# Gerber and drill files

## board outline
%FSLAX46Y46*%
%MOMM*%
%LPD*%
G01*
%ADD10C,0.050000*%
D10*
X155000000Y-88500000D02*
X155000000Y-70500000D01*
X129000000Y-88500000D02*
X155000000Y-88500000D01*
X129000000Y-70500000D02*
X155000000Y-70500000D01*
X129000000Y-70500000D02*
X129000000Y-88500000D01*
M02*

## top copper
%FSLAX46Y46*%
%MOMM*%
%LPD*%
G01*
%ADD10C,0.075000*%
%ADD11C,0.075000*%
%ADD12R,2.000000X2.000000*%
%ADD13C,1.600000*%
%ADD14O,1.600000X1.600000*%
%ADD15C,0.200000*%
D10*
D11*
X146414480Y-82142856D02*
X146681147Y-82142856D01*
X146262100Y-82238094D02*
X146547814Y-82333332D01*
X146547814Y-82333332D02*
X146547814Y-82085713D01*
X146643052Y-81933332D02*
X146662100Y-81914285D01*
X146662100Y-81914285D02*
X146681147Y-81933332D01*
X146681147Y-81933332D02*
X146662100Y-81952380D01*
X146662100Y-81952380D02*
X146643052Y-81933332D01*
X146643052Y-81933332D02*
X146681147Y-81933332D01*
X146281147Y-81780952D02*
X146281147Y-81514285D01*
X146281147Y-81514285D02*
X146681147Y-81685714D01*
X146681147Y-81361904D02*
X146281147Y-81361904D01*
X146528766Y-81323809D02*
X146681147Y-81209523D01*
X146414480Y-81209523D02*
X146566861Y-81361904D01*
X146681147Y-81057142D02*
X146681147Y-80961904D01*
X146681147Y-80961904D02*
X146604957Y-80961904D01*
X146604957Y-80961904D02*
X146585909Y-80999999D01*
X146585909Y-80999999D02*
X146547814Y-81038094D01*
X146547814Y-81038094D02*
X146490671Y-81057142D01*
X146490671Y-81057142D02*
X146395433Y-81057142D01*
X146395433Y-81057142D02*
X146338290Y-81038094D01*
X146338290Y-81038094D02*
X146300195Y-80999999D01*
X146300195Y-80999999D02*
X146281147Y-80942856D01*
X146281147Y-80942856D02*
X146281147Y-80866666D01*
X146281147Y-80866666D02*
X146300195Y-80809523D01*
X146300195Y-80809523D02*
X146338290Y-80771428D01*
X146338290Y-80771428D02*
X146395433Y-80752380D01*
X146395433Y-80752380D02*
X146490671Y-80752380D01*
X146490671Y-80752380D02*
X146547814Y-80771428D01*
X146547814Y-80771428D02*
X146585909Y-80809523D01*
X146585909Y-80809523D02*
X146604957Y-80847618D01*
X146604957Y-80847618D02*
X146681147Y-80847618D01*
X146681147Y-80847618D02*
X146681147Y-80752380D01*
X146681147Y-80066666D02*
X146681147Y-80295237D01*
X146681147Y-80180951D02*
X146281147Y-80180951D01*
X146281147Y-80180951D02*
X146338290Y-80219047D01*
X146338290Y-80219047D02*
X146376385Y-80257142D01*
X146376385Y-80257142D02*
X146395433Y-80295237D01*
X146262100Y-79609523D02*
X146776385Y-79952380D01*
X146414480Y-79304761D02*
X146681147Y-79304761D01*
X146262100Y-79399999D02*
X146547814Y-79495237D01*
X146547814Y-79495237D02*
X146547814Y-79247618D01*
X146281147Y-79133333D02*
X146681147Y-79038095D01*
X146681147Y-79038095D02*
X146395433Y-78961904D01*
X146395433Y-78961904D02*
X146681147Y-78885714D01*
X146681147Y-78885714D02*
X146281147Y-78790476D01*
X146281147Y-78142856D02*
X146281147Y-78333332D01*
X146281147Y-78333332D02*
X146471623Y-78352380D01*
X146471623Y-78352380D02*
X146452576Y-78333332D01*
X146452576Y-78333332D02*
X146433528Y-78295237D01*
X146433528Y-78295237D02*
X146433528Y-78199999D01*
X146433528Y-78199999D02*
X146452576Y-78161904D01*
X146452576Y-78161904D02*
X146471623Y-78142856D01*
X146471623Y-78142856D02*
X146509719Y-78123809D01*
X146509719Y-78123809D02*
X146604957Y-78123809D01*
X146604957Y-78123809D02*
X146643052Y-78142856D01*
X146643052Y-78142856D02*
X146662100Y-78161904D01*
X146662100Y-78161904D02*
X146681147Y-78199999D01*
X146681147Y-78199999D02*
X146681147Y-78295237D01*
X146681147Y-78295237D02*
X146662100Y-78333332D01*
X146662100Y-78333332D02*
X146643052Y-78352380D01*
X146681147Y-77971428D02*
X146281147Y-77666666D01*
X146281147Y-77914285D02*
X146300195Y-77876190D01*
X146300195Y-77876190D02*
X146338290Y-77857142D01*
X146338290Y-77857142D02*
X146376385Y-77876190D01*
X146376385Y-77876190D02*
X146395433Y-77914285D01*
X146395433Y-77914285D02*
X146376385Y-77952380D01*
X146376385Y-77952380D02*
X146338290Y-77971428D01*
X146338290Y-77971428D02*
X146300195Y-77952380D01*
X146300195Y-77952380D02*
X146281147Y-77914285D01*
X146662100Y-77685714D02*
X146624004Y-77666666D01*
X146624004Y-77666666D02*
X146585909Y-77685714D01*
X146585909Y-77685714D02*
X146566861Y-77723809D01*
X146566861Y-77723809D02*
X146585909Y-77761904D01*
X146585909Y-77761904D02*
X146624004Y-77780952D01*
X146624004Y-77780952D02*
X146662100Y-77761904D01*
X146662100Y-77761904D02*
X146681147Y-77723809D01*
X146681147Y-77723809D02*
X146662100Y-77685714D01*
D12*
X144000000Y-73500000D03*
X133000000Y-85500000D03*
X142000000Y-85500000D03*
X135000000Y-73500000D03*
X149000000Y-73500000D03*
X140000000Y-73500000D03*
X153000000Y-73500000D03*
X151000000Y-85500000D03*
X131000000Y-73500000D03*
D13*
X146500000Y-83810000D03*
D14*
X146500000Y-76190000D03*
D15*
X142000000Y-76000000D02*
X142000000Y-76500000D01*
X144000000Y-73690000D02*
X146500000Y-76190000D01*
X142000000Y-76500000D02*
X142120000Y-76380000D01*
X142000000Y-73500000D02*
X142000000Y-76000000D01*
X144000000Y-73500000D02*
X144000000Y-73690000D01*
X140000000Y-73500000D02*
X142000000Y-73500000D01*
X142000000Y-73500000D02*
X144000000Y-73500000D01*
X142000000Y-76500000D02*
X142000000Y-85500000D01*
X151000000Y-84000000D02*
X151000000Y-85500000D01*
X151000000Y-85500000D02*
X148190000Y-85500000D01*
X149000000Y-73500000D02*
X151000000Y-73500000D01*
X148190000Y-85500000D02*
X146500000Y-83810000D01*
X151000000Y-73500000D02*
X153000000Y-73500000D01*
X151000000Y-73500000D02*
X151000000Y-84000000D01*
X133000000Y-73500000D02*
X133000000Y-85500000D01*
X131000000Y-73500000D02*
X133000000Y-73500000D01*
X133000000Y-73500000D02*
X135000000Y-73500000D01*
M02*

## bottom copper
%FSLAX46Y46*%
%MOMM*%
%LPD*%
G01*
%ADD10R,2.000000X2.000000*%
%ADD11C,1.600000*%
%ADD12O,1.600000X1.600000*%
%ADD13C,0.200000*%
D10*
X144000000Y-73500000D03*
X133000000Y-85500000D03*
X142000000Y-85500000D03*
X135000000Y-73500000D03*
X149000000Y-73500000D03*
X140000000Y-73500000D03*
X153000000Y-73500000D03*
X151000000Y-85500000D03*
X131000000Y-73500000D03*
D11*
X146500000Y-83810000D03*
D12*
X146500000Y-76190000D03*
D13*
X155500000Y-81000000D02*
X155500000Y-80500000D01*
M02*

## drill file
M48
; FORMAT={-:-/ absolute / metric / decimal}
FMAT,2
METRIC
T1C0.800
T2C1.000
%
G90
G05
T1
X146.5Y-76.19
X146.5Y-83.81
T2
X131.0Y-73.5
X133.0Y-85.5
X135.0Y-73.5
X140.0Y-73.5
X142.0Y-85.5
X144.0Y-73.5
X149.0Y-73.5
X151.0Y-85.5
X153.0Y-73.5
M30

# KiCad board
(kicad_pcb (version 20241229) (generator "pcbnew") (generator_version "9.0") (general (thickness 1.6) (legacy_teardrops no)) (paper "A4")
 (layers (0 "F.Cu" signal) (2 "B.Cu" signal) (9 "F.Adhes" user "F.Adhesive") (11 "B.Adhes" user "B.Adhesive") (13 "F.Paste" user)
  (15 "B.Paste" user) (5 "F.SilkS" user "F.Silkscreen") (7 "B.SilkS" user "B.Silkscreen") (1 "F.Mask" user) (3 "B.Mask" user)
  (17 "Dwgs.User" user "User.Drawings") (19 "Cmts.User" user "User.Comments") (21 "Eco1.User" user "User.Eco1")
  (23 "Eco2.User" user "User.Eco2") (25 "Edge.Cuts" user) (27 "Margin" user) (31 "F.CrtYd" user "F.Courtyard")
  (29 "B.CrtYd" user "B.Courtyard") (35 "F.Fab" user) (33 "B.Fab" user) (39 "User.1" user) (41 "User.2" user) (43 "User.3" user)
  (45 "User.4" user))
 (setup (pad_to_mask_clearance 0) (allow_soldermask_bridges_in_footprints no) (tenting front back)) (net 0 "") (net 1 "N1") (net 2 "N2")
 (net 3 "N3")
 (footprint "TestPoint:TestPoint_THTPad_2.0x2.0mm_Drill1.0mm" (layer "F.Cu") (at 144 73.5)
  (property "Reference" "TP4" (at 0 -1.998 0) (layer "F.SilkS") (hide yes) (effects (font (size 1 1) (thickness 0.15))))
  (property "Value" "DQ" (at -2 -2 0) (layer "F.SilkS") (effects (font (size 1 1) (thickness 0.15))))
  (pad "1" thru_hole rect (at 0 0) (size 2 2) (drill 1) (layers "*.Cu" "*.Mask") (remove_unused_layers no) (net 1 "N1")))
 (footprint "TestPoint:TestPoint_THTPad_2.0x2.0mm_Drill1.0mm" (layer "F.Cu") (at 133 85.5)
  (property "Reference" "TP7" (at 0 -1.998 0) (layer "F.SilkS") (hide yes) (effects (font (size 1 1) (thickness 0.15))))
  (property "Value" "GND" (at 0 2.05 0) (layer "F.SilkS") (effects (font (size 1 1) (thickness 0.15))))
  (pad "1" thru_hole rect (at 0 0) (size 2 2) (drill 1) (layers "*.Cu" "*.Mask") (remove_unused_layers no) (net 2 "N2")))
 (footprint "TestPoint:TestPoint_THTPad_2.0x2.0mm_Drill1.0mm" (layer "F.Cu") (at 142 85.5)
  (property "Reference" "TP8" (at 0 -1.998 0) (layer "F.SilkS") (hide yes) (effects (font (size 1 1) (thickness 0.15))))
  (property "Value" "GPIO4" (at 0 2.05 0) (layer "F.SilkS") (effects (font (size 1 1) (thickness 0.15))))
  (pad "1" thru_hole rect (at 0 0) (size 2 2) (drill 1) (layers "*.Cu" "*.Mask") (remove_unused_layers no) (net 1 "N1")))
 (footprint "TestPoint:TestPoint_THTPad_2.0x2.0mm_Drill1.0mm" (layer "F.Cu") (at 135 73.5)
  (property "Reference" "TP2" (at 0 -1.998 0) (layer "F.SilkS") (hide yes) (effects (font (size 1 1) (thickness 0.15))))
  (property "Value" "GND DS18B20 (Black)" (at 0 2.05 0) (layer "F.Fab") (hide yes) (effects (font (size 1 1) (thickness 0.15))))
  (pad "1" thru_hole rect (at 0 0) (size 2 2) (drill 1) (layers "*.Cu" "*.Mask") (remove_unused_layers no) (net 2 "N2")))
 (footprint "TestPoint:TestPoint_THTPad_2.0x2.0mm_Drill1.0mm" (layer "F.Cu") (at 149 73.5)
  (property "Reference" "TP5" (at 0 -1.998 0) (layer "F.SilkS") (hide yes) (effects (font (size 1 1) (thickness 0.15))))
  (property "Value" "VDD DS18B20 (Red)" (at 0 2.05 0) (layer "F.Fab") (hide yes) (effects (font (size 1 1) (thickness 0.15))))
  (pad "1" thru_hole rect (at 0 0) (size 2 2) (drill 1) (layers "*.Cu" "*.Mask") (remove_unused_layers no) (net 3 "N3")))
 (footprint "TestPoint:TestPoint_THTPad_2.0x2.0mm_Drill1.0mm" (layer "F.Cu") (at 140 73.5)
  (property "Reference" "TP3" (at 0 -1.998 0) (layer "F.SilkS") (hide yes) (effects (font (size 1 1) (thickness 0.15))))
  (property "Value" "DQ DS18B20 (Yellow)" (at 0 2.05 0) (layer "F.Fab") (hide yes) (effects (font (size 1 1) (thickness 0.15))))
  (pad "1" thru_hole rect (at 0 0) (size 2 2) (drill 1) (layers "*.Cu" "*.Mask") (remove_unused_layers no) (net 1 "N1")))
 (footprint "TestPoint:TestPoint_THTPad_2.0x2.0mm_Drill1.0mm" (layer "F.Cu") (at 153 73.5)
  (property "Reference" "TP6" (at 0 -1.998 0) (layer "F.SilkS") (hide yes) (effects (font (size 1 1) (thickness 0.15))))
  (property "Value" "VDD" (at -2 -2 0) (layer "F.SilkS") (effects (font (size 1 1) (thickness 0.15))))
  (pad "1" thru_hole rect (at 0 0) (size 2 2) (drill 1) (layers "*.Cu" "*.Mask") (remove_unused_layers no) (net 3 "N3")))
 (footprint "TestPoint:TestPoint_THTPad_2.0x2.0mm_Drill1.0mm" (layer "F.Cu") (at 151 85.5)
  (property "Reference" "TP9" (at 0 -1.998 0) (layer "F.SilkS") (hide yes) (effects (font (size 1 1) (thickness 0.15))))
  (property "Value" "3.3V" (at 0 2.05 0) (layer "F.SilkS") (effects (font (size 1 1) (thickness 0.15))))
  (pad "1" thru_hole rect (at 0 0) (size 2 2) (drill 1) (layers "*.Cu" "*.Mask") (remove_unused_layers no) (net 3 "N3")))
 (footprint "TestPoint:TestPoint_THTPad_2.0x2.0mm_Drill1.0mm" (layer "F.Cu") (at 131 73.5)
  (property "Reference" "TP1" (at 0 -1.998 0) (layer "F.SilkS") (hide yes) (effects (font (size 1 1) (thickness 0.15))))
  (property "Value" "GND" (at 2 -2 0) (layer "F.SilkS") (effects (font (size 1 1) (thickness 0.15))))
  (pad "1" thru_hole rect (at 0 0) (size 2 2) (drill 1) (layers "*.Cu" "*.Mask") (remove_unused_layers no) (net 2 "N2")))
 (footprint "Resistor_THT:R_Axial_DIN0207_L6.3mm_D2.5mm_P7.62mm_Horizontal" (layer "F.Cu") (at 146.5 83.81 90)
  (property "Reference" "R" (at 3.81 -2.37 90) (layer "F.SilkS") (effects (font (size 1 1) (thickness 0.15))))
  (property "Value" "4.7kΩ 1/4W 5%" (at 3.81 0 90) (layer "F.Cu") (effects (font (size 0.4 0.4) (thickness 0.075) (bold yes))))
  (pad "1" thru_hole circle (at 0 0 90) (size 1.6 1.6) (drill 0.8) (layers "*.Cu" "*.Mask") (remove_unused_layers no) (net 3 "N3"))
  (pad "2" thru_hole oval (at 7.62 0 90) (size 1.6 1.6) (drill 0.8) (layers "*.Cu" "*.Mask") (remove_unused_layers no) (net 1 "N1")))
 (gr_line (start 155 88.5) (end 155 70.5) (stroke (width 0.05) (type default)) (layer "Edge.Cuts"))
 (gr_line (start 129 88.5) (end 155 88.5) (stroke (width 0.05) (type default)) (layer "Edge.Cuts"))
 (gr_line (start 129 70.5) (end 155 70.5) (stroke (width 0.05) (type default)) (layer "Edge.Cuts"))
 (gr_line (start 129 70.5) (end 129 88.5) (stroke (width 0.05) (type default)) (layer "Edge.Cuts"))
 (segment (start 142 76) (end 142 76.5) (width 0.2) (layer "F.Cu") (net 1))
 (segment (start 144 73.69) (end 146.5 76.19) (width 0.2) (layer "F.Cu") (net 1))
 (segment (start 142 76.5) (end 142.12 76.38) (width 0.2) (layer "F.Cu") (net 1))
 (segment (start 142 73.5) (end 142 76) (width 0.2) (layer "F.Cu") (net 1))
 (segment (start 144 73.5) (end 144 73.69) (width 0.2) (layer "F.Cu") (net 1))
 (segment (start 140 73.5) (end 142 73.5) (width 0.2) (layer "F.Cu") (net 1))
 (segment (start 142 73.5) (end 144 73.5) (width 0.2) (layer "F.Cu") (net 1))
 (segment (start 142 76.5) (end 142 85.5) (width 0.2) (layer "F.Cu") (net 1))
 (segment (start 155.5 81) (end 155.5 80.5) (width 0.2) (layer "B.Cu") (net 1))
 (segment (start 151 84) (end 151 85.5) (width 0.2) (layer "F.Cu") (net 3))
 (segment (start 151 85.5) (end 148.19 85.5) (width 0.2) (layer "F.Cu") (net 3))
 (segment (start 149 73.5) (end 151 73.5) (width 0.2) (layer "F.Cu") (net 3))
 (segment (start 148.19 85.5) (end 146.5 83.81) (width 0.2) (layer "F.Cu") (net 3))
 (segment (start 151 73.5) (end 153 73.5) (width 0.2) (layer "F.Cu") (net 3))
 (segment (start 151 73.5) (end 151 84) (width 0.2) (layer "F.Cu") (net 3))
 (segment (start 133 73.5) (end 133 85.5) (width 0.2) (layer "F.Cu") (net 2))
 (segment (start 131 73.5) (end 133 73.5) (width 0.2) (layer "F.Cu") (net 2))
 (segment (start 133 73.5) (end 135 73.5) (width 0.2) (layer "F.Cu") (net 2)))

